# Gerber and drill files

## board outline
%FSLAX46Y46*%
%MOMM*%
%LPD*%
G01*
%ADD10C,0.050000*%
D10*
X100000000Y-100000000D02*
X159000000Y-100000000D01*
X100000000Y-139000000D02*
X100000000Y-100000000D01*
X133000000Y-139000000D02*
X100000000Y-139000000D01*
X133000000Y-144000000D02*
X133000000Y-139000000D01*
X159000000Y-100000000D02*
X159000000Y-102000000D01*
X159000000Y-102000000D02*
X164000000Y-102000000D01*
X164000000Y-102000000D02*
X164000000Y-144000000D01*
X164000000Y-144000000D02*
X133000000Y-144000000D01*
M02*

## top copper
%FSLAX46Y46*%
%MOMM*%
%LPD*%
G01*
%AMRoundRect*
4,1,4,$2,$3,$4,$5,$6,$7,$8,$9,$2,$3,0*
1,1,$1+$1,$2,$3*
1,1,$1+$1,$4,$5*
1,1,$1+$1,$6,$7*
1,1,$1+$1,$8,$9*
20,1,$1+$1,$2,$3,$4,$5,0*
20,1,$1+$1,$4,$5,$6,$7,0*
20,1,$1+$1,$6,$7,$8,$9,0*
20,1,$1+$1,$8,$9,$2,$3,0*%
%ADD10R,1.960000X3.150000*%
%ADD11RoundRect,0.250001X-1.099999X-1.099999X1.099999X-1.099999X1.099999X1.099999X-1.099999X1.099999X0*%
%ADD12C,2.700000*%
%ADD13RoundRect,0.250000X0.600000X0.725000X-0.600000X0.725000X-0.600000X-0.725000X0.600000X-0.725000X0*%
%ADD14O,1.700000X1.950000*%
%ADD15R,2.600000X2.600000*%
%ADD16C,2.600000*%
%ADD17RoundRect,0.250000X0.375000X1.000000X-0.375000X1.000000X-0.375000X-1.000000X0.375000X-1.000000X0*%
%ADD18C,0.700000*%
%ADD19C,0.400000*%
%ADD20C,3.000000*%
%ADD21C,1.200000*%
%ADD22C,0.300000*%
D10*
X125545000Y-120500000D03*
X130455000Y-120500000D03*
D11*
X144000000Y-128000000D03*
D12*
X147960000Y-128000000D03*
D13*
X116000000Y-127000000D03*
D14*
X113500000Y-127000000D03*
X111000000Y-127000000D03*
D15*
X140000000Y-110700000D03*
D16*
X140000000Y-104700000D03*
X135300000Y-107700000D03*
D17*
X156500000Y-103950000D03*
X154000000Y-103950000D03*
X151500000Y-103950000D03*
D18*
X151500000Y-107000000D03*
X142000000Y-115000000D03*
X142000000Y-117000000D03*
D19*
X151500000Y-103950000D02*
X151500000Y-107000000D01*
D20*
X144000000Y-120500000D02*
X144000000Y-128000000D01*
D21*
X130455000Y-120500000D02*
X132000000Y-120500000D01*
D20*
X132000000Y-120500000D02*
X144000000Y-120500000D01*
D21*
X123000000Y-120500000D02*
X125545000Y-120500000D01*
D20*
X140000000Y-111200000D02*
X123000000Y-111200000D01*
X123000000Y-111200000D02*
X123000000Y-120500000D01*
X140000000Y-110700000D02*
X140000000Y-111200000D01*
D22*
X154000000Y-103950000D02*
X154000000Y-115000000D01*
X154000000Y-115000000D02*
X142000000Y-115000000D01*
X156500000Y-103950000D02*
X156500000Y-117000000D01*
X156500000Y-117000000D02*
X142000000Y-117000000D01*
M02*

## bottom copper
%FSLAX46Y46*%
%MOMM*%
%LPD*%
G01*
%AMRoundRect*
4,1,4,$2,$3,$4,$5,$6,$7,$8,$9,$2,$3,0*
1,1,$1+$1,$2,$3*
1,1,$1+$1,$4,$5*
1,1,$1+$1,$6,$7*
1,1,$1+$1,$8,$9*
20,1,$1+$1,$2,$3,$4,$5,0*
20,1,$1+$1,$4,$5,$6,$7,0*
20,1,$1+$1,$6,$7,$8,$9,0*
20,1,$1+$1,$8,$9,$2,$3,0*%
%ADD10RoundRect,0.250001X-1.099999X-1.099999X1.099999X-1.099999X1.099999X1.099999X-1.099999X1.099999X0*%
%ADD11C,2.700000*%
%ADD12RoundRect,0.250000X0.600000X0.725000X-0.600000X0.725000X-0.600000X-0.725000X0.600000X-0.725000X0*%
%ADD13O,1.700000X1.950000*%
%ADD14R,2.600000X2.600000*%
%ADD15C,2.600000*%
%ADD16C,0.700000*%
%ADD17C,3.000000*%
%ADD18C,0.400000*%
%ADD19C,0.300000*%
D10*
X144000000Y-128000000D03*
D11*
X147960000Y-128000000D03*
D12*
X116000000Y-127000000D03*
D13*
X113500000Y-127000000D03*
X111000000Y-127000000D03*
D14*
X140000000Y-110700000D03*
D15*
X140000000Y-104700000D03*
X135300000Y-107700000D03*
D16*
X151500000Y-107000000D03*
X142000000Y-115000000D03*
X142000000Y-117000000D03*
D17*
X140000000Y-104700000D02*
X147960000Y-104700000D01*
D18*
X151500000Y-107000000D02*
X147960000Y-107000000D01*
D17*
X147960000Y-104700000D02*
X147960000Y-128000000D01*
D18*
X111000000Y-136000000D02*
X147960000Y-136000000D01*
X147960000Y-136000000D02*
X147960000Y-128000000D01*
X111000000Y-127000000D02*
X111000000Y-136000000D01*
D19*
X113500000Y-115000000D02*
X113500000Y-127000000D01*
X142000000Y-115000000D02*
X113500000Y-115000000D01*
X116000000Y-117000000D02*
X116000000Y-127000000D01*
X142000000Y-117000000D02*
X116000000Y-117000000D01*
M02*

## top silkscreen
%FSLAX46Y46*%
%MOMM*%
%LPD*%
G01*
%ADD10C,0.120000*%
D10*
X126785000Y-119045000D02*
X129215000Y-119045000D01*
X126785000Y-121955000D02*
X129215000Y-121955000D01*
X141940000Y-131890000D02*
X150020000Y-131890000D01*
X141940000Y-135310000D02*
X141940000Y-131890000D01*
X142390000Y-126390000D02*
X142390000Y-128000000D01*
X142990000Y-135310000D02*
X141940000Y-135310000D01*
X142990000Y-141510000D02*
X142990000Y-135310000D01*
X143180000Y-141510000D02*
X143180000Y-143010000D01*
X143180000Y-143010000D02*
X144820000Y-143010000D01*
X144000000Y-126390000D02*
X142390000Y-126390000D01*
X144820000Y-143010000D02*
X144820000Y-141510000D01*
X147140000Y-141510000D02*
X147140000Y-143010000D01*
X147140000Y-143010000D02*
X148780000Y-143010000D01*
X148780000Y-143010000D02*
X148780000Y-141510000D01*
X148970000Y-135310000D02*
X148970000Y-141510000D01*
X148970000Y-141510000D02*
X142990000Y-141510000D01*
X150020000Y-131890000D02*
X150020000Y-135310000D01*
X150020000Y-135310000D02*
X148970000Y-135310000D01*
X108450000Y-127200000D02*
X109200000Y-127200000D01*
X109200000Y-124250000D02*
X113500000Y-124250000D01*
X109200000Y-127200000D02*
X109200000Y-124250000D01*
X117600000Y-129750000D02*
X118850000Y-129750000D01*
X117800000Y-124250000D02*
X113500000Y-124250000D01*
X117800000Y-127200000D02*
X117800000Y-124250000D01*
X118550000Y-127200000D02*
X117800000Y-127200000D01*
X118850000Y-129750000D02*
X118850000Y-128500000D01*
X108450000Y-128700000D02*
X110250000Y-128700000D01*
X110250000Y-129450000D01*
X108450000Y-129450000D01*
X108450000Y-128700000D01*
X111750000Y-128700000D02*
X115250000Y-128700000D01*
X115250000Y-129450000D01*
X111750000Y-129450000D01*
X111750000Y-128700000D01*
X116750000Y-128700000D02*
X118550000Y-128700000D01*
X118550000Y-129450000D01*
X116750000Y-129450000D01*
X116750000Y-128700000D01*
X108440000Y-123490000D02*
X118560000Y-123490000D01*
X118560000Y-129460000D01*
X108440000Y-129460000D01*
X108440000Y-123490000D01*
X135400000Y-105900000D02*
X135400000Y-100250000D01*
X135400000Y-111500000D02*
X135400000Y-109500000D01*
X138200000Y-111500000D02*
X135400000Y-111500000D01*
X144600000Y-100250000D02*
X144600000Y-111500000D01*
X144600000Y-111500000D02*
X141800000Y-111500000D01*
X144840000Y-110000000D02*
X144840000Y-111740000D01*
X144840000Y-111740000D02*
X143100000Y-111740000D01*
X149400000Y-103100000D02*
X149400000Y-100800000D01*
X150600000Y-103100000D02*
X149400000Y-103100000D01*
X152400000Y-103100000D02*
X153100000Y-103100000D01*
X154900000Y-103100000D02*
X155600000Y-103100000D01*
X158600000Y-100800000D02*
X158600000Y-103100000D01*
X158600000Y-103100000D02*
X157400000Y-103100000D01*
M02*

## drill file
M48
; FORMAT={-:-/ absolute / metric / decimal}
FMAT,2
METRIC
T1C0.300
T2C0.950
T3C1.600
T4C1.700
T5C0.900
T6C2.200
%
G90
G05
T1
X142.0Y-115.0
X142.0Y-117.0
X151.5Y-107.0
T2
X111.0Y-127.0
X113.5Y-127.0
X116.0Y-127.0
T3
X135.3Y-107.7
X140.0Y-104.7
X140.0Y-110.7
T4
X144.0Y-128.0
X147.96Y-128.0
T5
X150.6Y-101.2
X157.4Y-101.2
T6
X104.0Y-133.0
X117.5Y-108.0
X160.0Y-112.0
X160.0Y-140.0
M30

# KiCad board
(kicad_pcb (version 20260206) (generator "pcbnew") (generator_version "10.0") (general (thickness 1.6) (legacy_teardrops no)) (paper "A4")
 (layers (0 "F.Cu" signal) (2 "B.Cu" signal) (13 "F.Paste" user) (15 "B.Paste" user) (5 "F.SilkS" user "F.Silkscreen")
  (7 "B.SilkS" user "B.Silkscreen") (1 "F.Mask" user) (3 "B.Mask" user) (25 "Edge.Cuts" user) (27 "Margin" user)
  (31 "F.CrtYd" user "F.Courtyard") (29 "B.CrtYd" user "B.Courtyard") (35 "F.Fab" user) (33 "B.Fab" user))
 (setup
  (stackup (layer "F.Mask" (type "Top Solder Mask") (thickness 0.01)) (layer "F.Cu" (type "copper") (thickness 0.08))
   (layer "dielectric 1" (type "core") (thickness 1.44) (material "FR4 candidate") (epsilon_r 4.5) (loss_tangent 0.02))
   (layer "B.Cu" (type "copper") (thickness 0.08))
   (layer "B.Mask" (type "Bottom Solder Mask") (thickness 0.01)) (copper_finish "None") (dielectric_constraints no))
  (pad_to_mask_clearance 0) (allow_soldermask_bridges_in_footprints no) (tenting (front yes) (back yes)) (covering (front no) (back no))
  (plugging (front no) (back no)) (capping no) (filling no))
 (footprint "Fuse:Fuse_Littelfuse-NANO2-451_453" (layer "F.Cu") (at 128 120.5)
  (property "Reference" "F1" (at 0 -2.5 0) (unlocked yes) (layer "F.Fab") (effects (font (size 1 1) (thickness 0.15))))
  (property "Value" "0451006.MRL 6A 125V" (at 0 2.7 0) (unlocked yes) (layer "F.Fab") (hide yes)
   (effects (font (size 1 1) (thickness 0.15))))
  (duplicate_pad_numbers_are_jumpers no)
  (fp_line (start -1.215 -1.455) (end 1.215 -1.455) (stroke (width 0.12) (type solid)) (layer "F.SilkS"))
  (fp_line (start -1.215 1.455) (end 1.215 1.455) (stroke (width 0.12) (type solid)) (layer "F.SilkS"))
  (pad "1" smd rect (at -2.455 0) (size 1.96 3.15) (layers "F.Cu" "F.Mask" "F.Paste") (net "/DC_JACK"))
  (pad "2" smd rect (at 2.455 0) (size 1.96 3.15) (layers "F.Cu" "F.Mask" "F.Paste") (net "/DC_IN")))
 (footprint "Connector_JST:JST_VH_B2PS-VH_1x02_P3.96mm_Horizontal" (layer "F.Cu") (at 144 128)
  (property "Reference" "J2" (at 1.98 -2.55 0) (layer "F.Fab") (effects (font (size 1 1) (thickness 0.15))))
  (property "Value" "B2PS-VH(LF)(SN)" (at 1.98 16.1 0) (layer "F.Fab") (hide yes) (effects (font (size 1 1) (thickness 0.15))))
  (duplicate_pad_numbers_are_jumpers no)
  (fp_line (start -2.06 3.89) (end 6.02 3.89) (stroke (width 0.12) (type solid)) (layer "F.SilkS"))
  (fp_line (start -2.06 7.31) (end -2.06 3.89) (stroke (width 0.12) (type solid)) (layer "F.SilkS"))
  (fp_line (start -1.61 -1.61) (end -1.61 0) (stroke (width 0.12) (type solid)) (layer "F.SilkS"))
  (fp_line (start -1.01 7.31) (end -2.06 7.31) (stroke (width 0.12) (type solid)) (layer "F.SilkS"))
  (fp_line (start -1.01 13.51) (end -1.01 7.31) (stroke (width 0.12) (type solid)) (layer "F.SilkS"))
  (fp_line (start -0.82 13.51) (end -0.82 15.01) (stroke (width 0.12) (type solid)) (layer "F.SilkS"))
  (fp_line (start -0.82 15.01) (end 0.82 15.01) (stroke (width 0.12) (type solid)) (layer "F.SilkS"))
  (fp_line (start 0 -1.61) (end -1.61 -1.61) (stroke (width 0.12) (type solid)) (layer "F.SilkS"))
  (fp_line (start 0.82 15.01) (end 0.82 13.51) (stroke (width 0.12) (type solid)) (layer "F.SilkS"))
  (fp_line (start 3.14 13.51) (end 3.14 15.01) (stroke (width 0.12) (type solid)) (layer "F.SilkS"))
  (fp_line (start 3.14 15.01) (end 4.78 15.01) (stroke (width 0.12) (type solid)) (layer "F.SilkS"))
  (fp_line (start 4.78 15.01) (end 4.78 13.51) (stroke (width 0.12) (type solid)) (layer "F.SilkS"))
  (fp_line (start 4.97 7.31) (end 4.97 13.51) (stroke (width 0.12) (type solid)) (layer "F.SilkS"))
  (fp_line (start 4.97 13.51) (end -1.01 13.51) (stroke (width 0.12) (type solid)) (layer "F.SilkS"))
  (fp_line (start 6.02 3.89) (end 6.02 7.31) (stroke (width 0.12) (type solid)) (layer "F.SilkS"))
  (fp_line (start 6.02 7.31) (end 4.97 7.31) (stroke (width 0.12) (type solid)) (layer "F.SilkS"))
  (pad "1" thru_hole roundrect (at 0 0) (size 2.7 2.7) (drill 1.7) (layers "*.Cu" "*.Mask") (remove_unused_layers no)
   (roundrect_rratio 0.092593) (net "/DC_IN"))
  (pad "2" thru_hole circle (at 3.96 0) (size 2.7 2.7) (drill 1.7) (layers "*.Cu" "*.Mask") (remove_unused_layers no) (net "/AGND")))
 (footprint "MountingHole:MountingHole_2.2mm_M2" (layer "F.Cu") (at 104 133)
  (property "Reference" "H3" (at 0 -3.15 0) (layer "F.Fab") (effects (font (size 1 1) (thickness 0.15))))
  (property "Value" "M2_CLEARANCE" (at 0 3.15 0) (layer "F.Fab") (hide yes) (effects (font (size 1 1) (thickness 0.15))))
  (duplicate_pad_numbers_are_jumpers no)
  (pad "" np_thru_hole circle (at 0 0) (size 2.2 2.2) (drill 2.2) (layers "*.Cu" "*.Mask")))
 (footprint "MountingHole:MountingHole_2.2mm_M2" (layer "F.Cu") (at 160 112)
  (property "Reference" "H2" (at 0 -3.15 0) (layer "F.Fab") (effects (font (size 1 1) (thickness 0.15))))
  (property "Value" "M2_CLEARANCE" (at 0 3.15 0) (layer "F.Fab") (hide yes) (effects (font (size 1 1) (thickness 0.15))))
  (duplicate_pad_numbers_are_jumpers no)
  (pad "" np_thru_hole circle (at 0 0) (size 2.2 2.2) (drill 2.2) (layers "*.Cu" "*.Mask")))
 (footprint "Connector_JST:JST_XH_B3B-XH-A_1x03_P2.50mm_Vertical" (layer "F.Cu") (at 116 127 180)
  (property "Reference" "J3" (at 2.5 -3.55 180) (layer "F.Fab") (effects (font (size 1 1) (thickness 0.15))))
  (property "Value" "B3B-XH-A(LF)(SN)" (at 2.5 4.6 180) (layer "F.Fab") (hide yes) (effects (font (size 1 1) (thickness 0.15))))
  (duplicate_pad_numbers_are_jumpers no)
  (fp_line (start 7.55 -0.2) (end 6.8 -0.2) (stroke (width 0.12) (type solid)) (layer "F.SilkS"))
  (fp_line (start 6.8 2.75) (end 2.5 2.75) (stroke (width 0.12) (type solid)) (layer "F.SilkS"))
  (fp_line (start 6.8 -0.2) (end 6.8 2.75) (stroke (width 0.12) (type solid)) (layer "F.SilkS"))
  (fp_line (start -1.6 -2.75) (end -2.85 -2.75) (stroke (width 0.12) (type solid)) (layer "F.SilkS"))
  (fp_line (start -1.8 2.75) (end 2.5 2.75) (stroke (width 0.12) (type solid)) (layer "F.SilkS"))
  (fp_line (start -1.8 -0.2) (end -1.8 2.75) (stroke (width 0.12) (type solid)) (layer "F.SilkS"))
  (fp_line (start -2.55 -0.2) (end -1.8 -0.2) (stroke (width 0.12) (type solid)) (layer "F.SilkS"))
  (fp_line (start -2.85 -2.75) (end -2.85 -1.5) (stroke (width 0.12) (type solid)) (layer "F.SilkS"))
  (fp_rect (start 5.75 -2.45) (end 7.55 -1.7) (stroke (width 0.12) (type solid)) (fill no) (layer "F.SilkS"))
  (fp_rect (start 0.75 -2.45) (end 4.25 -1.7) (stroke (width 0.12) (type solid)) (fill no) (layer "F.SilkS"))
  (fp_rect (start -2.55 -2.45) (end -0.75 -1.7) (stroke (width 0.12) (type solid)) (fill no) (layer "F.SilkS"))
  (fp_rect (start -2.56 -2.46) (end 7.56 3.51) (stroke (width 0.12) (type solid)) (fill no) (layer "F.SilkS"))
  (pad "1" thru_hole roundrect (at 0 0 180) (size 1.7 1.95) (drill 0.95) (layers "*.Cu" "*.Mask") (remove_unused_layers no)
   (roundrect_rratio 0.147059) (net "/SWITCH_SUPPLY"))
  (pad "2" thru_hole oval (at 2.5 0 180) (size 1.7 1.95) (drill 0.95) (layers "*.Cu" "*.Mask") (remove_unused_layers no) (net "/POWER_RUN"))
  (pad "3" thru_hole oval (at 5 0 180) (size 1.7 1.95) (drill 0.95) (layers "*.Cu" "*.Mask") (remove_unused_layers no) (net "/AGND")))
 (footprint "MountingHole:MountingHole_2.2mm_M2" (layer "F.Cu") (at 160 140)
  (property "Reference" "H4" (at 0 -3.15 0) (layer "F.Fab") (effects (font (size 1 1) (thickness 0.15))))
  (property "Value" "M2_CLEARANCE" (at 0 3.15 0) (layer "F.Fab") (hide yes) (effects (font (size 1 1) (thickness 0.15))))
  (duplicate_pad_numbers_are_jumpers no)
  (pad "" np_thru_hole circle (at 0 0) (size 2.2 2.2) (drill 2.2) (layers "*.Cu" "*.Mask")))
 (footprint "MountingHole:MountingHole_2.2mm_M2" (layer "F.Cu") (at 117.5 108)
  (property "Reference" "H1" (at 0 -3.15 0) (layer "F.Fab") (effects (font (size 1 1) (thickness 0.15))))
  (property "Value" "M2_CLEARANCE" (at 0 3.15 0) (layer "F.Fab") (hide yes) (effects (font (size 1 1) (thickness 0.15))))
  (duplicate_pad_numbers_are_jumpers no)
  (pad "" np_thru_hole circle (at 0 0) (size 2.2 2.2) (drill 2.2) (layers "*.Cu" "*.Mask")))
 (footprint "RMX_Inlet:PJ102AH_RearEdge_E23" (layer "F.Cu") (at 140 110.7 180)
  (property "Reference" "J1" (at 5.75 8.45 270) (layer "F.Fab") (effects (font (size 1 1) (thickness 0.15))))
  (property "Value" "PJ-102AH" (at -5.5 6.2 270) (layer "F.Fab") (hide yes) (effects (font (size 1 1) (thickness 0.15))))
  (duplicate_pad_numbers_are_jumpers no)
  (fp_line (start 4.6 4.8) (end 4.6 10.45) (stroke (width 0.12) (type solid)) (layer "F.SilkS"))
  (fp_line (start 4.6 -0.8) (end 4.6 1.2) (stroke (width 0.12) (type solid)) (layer "F.SilkS"))
  (fp_line (start 1.8 -0.8) (end 4.6 -0.8) (stroke (width 0.12) (type solid)) (layer "F.SilkS"))
  (fp_line (start -4.6 10.45) (end -4.6 -0.8) (stroke (width 0.12) (type solid)) (layer "F.SilkS"))
  (fp_line (start -4.6 -0.8) (end -1.8 -0.8) (stroke (width 0.12) (type solid)) (layer "F.SilkS"))
  (fp_line (start -4.84 0.7) (end -4.84 -1.04) (stroke (width 0.12) (type solid)) (layer "F.SilkS"))
  (fp_line (start -4.84 -1.04) (end -3.1 -1.04) (stroke (width 0.12) (type solid)) (layer "F.SilkS"))
  (pad "1" thru_hole rect (at 0 0 180) (size 2.6 2.6) (drill 1.6) (layers "*.Cu" "*.Mask") (remove_unused_layers no) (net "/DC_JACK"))
  (pad "2" thru_hole circle (at 0 6 180) (size 2.6 2.6) (drill 1.6) (layers "*.Cu" "*.Mask") (remove_unused_layers no) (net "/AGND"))
  (pad "3" thru_hole circle (at 4.7 3 180) (size 2.6 2.6) (drill 1.6) (layers "*.Cu" "*.Mask") (remove_unused_layers no)
   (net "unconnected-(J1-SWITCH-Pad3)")))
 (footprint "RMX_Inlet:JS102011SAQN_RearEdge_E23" (layer "F.Cu") (at 154 101.2 180)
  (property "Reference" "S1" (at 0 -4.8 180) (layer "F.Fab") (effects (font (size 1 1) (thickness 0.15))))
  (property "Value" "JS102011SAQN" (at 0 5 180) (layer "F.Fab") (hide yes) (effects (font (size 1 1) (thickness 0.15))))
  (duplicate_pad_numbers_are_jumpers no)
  (fp_line (start 4.6 -1.9) (end 4.6 0.4) (stroke (width 0.12) (type solid)) (layer "F.SilkS"))
  (fp_line (start 3.4 -1.9) (end 4.6 -1.9) (stroke (width 0.12) (type solid)) (layer "F.SilkS"))
  (fp_line (start 1.6 -1.9) (end 0.9 -1.9) (stroke (width 0.12) (type solid)) (layer "F.SilkS"))
  (fp_line (start -0.9 -1.9) (end -1.6 -1.9) (stroke (width 0.12) (type solid)) (layer "F.SilkS"))
  (fp_line (start -4.6 0.4) (end -4.6 -1.9) (stroke (width 0.12) (type solid)) (layer "F.SilkS"))
  (fp_line (start -4.6 -1.9) (end -3.4 -1.9) (stroke (width 0.12) (type solid)) (layer "F.SilkS"))
  (pad "" np_thru_hole circle (at -3.4 0 180) (size 0.9 0.9) (drill 0.9) (layers "*.Cu" "*.Mask"))
  (pad "" np_thru_hole circle (at 3.4 0 180) (size 0.9 0.9) (drill 0.9) (layers "*.Cu" "*.Mask"))
  (pad "1" smd roundrect (at -2.5 -2.75 180) (size 1.25 2.5) (layers "F.Cu" "F.Mask" "F.Paste") (roundrect_rratio 0.2)
   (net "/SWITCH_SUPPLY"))
  (pad "2" smd roundrect (at 0 -2.75 180) (size 1.25 2.5) (layers "F.Cu" "F.Mask" "F.Paste") (roundrect_rratio 0.2) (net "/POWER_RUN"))
  (pad "3" smd roundrect (at 2.5 -2.75 180) (size 1.25 2.5) (layers "F.Cu" "F.Mask" "F.Paste") (roundrect_rratio 0.2) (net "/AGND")))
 (gr_line (start 100 100) (end 159 100) (stroke (width 0.05) (type default)) (layer "Edge.Cuts"))
 (gr_line (start 100 139) (end 100 100) (stroke (width 0.05) (type default)) (layer "Edge.Cuts"))
 (gr_line (start 133 139) (end 100 139) (stroke (width 0.05) (type default)) (layer "Edge.Cuts"))
 (gr_line (start 133 144) (end 133 139) (stroke (width 0.05) (type default)) (layer "Edge.Cuts"))
 (gr_line (start 159 100) (end 159 102) (stroke (width 0.05) (type default)) (layer "Edge.Cuts"))
 (gr_line (start 159 102) (end 164 102) (stroke (width 0.05) (type default)) (layer "Edge.Cuts"))
 (gr_line (start 164 102) (end 164 144) (stroke (width 0.05) (type default)) (layer "Edge.Cuts"))
 (gr_line (start 164 144) (end 133 144) (stroke (width 0.05) (type default)) (layer "Edge.Cuts"))
 (segment (start 151.5 103.95) (end 151.5 107) (width 0.4) (layer "F.Cu") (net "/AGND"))
 (via (at 151.5 107) (size 0.7) (drill 0.3) (layers "F.Cu" "B.Cu") (capping no) (covering (front no) (back no))
  (plugging (front no) (back no)) (filling no) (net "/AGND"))
 (segment (start 140 104.7) (end 147.96 104.7) (width 3) (layer "B.Cu") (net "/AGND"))
 (segment (start 151.5 107) (end 147.96 107) (width 0.4) (layer "B.Cu") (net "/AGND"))
 (segment (start 147.96 104.7) (end 147.96 128) (width 3) (layer "B.Cu") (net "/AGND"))
 (segment (start 111 136) (end 147.96 136) (width 0.4) (layer "B.Cu") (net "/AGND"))
 (segment (start 147.96 136) (end 147.96 128) (width 0.4) (layer "B.Cu") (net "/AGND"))
 (segment (start 111 127) (end 111 136) (width 0.4) (layer "B.Cu") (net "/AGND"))
 (segment (start 144 120.5) (end 144 128) (width 3) (layer "F.Cu") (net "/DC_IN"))
 (segment (start 130.455 120.5) (end 132 120.5) (width 1.2) (layer "F.Cu") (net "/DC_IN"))
 (segment (start 132 120.5) (end 144 120.5) (width 3) (layer "F.Cu") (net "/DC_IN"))
 (segment (start 123 120.5) (end 125.545 120.5) (width 1.2) (layer "F.Cu") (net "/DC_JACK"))
 (segment (start 140 111.2) (end 123 111.2) (width 3) (layer "F.Cu") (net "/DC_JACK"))
 (segment (start 123 111.2) (end 123 120.5) (width 3) (layer "F.Cu") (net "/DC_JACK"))
 (segment (start 140 110.7) (end 140 111.2) (width 3) (layer "F.Cu") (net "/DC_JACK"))
 (segment (start 154 103.95) (end 154 115) (width 0.3) (layer "F.Cu") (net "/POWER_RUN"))
 (segment (start 154 115) (end 142 115) (width 0.3) (layer "F.Cu") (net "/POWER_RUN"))
 (via (at 142 115) (size 0.7) (drill 0.3) (layers "F.Cu" "B.Cu") (capping no) (covering (front no) (back no))
  (plugging (front no) (back no)) (filling no) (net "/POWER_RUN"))
 (segment (start 113.5 115) (end 113.5 127) (width 0.3) (layer "B.Cu") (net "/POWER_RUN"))
 (segment (start 142 115) (end 113.5 115) (width 0.3) (layer "B.Cu") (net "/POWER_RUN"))
 (segment (start 156.5 103.95) (end 156.5 117) (width 0.3) (layer "F.Cu") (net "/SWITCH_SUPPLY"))
 (segment (start 156.5 117) (end 142 117) (width 0.3) (layer "F.Cu") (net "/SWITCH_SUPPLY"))
 (via (at 142 117) (size 0.7) (drill 0.3) (layers "F.Cu" "B.Cu") (capping no) (covering (front no) (back no))
  (plugging (front no) (back no)) (filling no) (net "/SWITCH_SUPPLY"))
 (segment (start 116 117) (end 116 127) (width 0.3) (layer "B.Cu") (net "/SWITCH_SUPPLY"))
 (segment (start 142 117) (end 116 117) (width 0.3) (layer "B.Cu") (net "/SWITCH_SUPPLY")))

